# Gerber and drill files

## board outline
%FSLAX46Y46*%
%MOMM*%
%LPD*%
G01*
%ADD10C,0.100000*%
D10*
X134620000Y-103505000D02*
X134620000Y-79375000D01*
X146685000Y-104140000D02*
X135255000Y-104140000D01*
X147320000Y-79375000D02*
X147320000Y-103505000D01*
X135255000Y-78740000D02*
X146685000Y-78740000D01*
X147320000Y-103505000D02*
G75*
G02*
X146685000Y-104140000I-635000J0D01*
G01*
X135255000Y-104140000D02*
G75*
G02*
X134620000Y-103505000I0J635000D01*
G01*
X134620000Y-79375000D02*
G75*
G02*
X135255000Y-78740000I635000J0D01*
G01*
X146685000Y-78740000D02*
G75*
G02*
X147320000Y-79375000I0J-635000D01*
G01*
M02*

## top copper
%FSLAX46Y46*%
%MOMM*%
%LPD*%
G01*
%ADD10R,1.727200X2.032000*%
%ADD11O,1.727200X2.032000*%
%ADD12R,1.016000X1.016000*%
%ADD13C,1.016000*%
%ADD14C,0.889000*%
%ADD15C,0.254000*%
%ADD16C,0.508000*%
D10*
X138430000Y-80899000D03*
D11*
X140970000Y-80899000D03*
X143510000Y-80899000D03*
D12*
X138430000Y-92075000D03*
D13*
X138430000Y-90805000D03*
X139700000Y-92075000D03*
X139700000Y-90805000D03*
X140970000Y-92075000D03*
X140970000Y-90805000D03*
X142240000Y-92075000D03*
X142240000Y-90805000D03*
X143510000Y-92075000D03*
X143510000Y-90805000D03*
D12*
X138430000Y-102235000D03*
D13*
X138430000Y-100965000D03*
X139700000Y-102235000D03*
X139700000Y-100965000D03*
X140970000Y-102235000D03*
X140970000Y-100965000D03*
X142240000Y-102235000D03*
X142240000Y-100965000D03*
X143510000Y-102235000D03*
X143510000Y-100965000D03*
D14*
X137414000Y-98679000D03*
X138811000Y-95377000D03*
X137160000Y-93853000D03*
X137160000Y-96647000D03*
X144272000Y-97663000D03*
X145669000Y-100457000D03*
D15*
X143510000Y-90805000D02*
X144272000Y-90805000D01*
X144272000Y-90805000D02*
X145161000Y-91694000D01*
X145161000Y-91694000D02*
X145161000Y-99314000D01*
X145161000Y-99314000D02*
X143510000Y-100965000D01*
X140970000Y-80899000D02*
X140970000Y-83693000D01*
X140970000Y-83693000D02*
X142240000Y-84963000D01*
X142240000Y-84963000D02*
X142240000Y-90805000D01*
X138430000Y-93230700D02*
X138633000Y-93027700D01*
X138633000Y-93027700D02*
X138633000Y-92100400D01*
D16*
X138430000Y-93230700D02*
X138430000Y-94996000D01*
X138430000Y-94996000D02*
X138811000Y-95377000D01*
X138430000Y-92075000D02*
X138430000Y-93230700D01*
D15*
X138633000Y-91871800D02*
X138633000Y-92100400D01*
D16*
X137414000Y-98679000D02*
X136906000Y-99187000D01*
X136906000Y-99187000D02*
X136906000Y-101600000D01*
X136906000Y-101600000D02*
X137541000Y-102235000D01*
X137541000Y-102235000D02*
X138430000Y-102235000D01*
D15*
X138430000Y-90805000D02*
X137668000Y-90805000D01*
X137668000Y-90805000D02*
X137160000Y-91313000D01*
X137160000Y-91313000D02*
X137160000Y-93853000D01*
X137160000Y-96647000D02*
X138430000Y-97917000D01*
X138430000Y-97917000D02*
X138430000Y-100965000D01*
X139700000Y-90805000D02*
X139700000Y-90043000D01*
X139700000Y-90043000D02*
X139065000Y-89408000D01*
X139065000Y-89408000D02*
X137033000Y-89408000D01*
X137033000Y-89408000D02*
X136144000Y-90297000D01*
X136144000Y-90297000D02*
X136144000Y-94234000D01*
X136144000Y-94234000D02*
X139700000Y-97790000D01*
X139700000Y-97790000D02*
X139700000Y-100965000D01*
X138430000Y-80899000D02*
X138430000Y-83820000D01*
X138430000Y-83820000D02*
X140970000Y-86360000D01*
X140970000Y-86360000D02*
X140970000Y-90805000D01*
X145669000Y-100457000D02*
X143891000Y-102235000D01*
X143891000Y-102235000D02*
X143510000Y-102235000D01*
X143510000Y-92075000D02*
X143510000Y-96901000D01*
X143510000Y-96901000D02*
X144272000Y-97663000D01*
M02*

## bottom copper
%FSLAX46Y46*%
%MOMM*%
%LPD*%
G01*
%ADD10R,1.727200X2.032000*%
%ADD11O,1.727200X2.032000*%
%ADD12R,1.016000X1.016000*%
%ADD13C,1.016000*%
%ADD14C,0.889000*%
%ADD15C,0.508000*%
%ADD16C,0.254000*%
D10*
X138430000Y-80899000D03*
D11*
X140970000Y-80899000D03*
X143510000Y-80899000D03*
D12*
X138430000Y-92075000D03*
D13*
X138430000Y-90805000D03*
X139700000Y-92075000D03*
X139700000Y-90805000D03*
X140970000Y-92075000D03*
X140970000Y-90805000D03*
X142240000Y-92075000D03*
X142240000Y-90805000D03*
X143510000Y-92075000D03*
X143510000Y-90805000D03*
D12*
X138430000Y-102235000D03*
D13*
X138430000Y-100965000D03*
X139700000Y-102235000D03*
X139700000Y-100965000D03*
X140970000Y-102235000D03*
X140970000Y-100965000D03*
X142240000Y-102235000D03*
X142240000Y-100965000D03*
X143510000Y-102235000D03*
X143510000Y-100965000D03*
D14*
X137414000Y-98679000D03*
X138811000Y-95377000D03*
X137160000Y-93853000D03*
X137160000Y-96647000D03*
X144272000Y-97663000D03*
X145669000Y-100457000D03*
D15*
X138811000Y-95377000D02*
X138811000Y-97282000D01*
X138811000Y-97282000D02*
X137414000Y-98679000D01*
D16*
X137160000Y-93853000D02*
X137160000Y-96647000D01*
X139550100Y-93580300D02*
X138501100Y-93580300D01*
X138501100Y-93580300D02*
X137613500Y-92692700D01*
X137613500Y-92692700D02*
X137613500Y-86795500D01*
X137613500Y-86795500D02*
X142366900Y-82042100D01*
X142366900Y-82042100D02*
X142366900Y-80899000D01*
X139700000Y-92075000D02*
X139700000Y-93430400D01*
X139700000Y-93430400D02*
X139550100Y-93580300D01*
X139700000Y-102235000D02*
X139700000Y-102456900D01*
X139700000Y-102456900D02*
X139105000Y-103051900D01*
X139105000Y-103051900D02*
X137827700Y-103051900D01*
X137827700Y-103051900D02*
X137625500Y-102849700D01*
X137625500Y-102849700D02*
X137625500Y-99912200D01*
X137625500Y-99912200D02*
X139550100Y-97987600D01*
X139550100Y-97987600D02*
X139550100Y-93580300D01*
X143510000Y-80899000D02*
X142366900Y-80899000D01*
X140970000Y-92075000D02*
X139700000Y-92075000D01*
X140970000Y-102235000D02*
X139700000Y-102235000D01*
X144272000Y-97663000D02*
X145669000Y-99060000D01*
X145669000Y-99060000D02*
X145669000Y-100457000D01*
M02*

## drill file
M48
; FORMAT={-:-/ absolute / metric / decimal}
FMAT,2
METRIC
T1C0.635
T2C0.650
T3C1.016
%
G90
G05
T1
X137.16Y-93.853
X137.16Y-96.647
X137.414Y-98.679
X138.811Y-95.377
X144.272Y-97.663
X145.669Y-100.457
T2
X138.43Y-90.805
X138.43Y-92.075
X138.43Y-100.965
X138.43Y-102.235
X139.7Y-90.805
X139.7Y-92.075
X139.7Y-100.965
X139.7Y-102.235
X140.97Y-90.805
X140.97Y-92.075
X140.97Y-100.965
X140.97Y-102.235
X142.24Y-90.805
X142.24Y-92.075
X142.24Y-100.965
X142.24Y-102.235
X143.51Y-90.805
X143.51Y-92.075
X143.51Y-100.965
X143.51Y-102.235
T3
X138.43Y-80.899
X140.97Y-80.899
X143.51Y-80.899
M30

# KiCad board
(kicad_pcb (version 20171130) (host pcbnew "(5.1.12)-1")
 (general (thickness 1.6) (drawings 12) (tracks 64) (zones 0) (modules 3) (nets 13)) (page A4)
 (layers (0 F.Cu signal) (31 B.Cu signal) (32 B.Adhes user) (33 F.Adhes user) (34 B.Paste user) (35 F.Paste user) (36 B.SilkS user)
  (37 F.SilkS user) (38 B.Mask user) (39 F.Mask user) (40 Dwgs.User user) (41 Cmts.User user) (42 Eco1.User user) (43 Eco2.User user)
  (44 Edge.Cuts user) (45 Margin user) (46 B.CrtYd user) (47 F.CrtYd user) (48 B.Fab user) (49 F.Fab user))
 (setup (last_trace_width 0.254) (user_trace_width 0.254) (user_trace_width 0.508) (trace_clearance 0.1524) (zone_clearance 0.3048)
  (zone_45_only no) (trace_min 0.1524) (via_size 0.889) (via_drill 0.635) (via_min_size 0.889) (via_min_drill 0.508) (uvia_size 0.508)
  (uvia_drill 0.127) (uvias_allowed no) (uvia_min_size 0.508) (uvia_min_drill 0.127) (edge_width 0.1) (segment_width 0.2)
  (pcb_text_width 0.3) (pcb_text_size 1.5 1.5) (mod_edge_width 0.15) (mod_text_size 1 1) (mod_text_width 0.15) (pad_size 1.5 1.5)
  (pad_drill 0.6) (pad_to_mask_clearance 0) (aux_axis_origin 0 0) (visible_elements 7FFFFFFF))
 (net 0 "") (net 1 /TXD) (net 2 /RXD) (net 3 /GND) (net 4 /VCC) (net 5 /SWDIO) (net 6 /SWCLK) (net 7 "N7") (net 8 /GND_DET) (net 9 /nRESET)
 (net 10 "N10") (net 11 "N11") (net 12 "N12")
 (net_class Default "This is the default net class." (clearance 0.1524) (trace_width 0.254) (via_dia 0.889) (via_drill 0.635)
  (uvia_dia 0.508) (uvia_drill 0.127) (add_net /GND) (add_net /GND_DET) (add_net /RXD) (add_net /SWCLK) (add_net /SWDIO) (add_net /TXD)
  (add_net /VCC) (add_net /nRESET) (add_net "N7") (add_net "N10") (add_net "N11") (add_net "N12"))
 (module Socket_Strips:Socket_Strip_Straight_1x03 (layer F.Cu) (at 140.97 80.899 180)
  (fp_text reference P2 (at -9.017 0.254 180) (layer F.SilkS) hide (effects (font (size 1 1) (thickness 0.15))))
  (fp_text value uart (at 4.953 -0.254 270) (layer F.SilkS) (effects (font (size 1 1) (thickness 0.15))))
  (pad 1 thru_hole rect (at 2.54 0) (size 1.7272 2.032) (drill 1.016) (layers *.Cu *.Mask F.SilkS) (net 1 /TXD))
  (pad 2 thru_hole oval (at 0 0) (size 1.7272 2.032) (drill 1.016) (layers *.Cu *.Mask F.SilkS) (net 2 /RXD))
  (pad 3 thru_hole oval (at -2.54 0) (size 1.7272 2.032) (drill 1.016) (layers *.Cu *.Mask F.SilkS) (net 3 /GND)))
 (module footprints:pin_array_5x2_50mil (layer F.Cu) (at 139.7 91.44)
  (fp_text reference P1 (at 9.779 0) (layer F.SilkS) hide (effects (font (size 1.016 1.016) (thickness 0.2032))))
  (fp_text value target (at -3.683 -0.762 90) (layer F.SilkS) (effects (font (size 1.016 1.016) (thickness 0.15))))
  (pad 1 thru_hole rect (at -1.27 0.635) (size 1.016 1.016) (drill 0.65) (layers *.Cu *.Mask F.SilkS) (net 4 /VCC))
  (pad 2 thru_hole circle (at -1.27 -0.635) (size 1.016 1.016) (drill 0.65) (layers *.Cu *.Mask F.SilkS) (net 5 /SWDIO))
  (pad 3 thru_hole circle (at 0 0.635) (size 1.016 1.016) (drill 0.65) (layers *.Cu *.Mask F.SilkS) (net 3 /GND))
  (pad 4 thru_hole circle (at 0 -0.635) (size 1.016 1.016) (drill 0.65) (layers *.Cu *.Mask F.SilkS) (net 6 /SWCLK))
  (pad 5 thru_hole circle (at 1.27 0.635) (size 1.016 1.016) (drill 0.65) (layers *.Cu *.Mask F.SilkS) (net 3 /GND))
  (pad 6 thru_hole circle (at 1.27 -0.635) (size 1.016 1.016) (drill 0.65) (layers *.Cu *.Mask F.SilkS) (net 1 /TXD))
  (pad 7 thru_hole circle (at 2.54 0.635) (size 1.016 1.016) (drill 0.65) (layers *.Cu *.Mask F.SilkS) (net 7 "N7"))
  (pad 8 thru_hole circle (at 2.54 -0.635) (size 1.016 1.016) (drill 0.65) (layers *.Cu *.Mask F.SilkS) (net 2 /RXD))
  (pad 9 thru_hole circle (at 3.81 0.635) (size 1.016 1.016) (drill 0.65) (layers *.Cu *.Mask F.SilkS) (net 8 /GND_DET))
  (pad 10 thru_hole circle (at 3.81 -0.635) (size 1.016 1.016) (drill 0.65) (layers *.Cu *.Mask F.SilkS) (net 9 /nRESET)))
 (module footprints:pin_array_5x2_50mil (layer F.Cu) (at 139.7 101.6)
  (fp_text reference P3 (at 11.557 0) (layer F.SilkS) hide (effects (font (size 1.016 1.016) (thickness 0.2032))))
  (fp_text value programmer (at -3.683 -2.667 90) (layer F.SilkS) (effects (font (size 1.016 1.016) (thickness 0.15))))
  (pad 1 thru_hole rect (at -1.27 0.635) (size 1.016 1.016) (drill 0.65) (layers *.Cu *.Mask F.SilkS) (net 4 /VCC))
  (pad 2 thru_hole circle (at -1.27 -0.635) (size 1.016 1.016) (drill 0.65) (layers *.Cu *.Mask F.SilkS) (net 5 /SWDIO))
  (pad 3 thru_hole circle (at 0 0.635) (size 1.016 1.016) (drill 0.65) (layers *.Cu *.Mask F.SilkS) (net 3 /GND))
  (pad 4 thru_hole circle (at 0 -0.635) (size 1.016 1.016) (drill 0.65) (layers *.Cu *.Mask F.SilkS) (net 6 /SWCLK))
  (pad 5 thru_hole circle (at 1.27 0.635) (size 1.016 1.016) (drill 0.65) (layers *.Cu *.Mask F.SilkS) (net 3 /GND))
  (pad 6 thru_hole circle (at 1.27 -0.635) (size 1.016 1.016) (drill 0.65) (layers *.Cu *.Mask F.SilkS) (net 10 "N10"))
  (pad 7 thru_hole circle (at 2.54 0.635) (size 1.016 1.016) (drill 0.65) (layers *.Cu *.Mask F.SilkS) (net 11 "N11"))
  (pad 8 thru_hole circle (at 2.54 -0.635) (size 1.016 1.016) (drill 0.65) (layers *.Cu *.Mask F.SilkS) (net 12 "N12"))
  (pad 9 thru_hole circle (at 3.81 0.635) (size 1.016 1.016) (drill 0.65) (layers *.Cu *.Mask F.SilkS) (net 8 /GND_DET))
  (pad 10 thru_hole circle (at 3.81 -0.635) (size 1.016 1.016) (drill 0.65) (layers *.Cu *.Mask F.SilkS) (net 9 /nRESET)))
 (gr_line (start 134.62 103.505) (end 134.62 79.375) (angle 90) (layer Edge.Cuts) (width 0.1))
 (gr_line (start 146.685 104.14) (end 135.255 104.14) (angle 90) (layer Edge.Cuts) (width 0.1))
 (gr_line (start 147.32 79.375) (end 147.32 103.505) (angle 90) (layer Edge.Cuts) (width 0.1))
 (gr_line (start 135.255 78.74) (end 146.685 78.74) (angle 90) (layer Edge.Cuts) (width 0.1))
 (gr_arc (start 146.685 103.505) (end 147.32 103.505) (angle 90) (layer Edge.Cuts) (width 0.1))
 (gr_arc (start 135.255 103.505) (end 135.255 104.14) (angle 90) (layer Edge.Cuts) (width 0.1))
 (gr_arc (start 135.255 79.375) (end 134.62 79.375) (angle 90) (layer Edge.Cuts) (width 0.1))
 (gr_arc (start 146.685 79.375) (end 146.685 78.74) (angle 90) (layer Edge.Cuts) (width 0.1))
 (segment (start 143.51 90.805) (end 144.272 90.805) (width 0.254) (layer F.Cu) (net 9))
 (segment (start 144.272 90.805) (end 145.161 91.694) (width 0.254) (layer F.Cu) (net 9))
 (segment (start 145.161 91.694) (end 145.161 99.314) (width 0.254) (layer F.Cu) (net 9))
 (segment (start 145.161 99.314) (end 143.51 100.965) (width 0.254) (layer F.Cu) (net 9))
 (segment (start 140.97 80.899) (end 140.97 83.693) (width 0.254) (layer F.Cu) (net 2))
 (segment (start 140.97 83.693) (end 142.24 84.963) (width 0.254) (layer F.Cu) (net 2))
 (segment (start 142.24 84.963) (end 142.24 90.805) (width 0.254) (layer F.Cu) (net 2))
 (segment (start 138.43 93.2307) (end 138.633 93.0277) (width 0.254) (layer F.Cu) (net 4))
 (segment (start 138.633 93.0277) (end 138.633 92.1004) (width 0.254) (layer F.Cu) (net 4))
 (segment (start 138.43 93.2307) (end 138.43 94.996) (width 0.508) (layer F.Cu) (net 4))
 (segment (start 138.43 94.996) (end 138.811 95.377) (width 0.508) (layer F.Cu) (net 4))
 (segment (start 138.43 92.075) (end 138.43 93.2307) (width 0.508) (layer F.Cu) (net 4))
 (segment (start 138.633 91.8718) (end 138.633 92.1004) (width 0.254) (layer F.Cu) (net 4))
 (segment (start 137.414 98.679) (end 136.906 99.187) (width 0.508) (layer F.Cu) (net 4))
 (segment (start 136.906 99.187) (end 136.906 101.6) (width 0.508) (layer F.Cu) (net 4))
 (segment (start 136.906 101.6) (end 137.541 102.235) (width 0.508) (layer F.Cu) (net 4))
 (segment (start 137.541 102.235) (end 138.43 102.235) (width 0.508) (layer F.Cu) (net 4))
 (segment (start 138.811 95.377) (end 138.811 97.282) (width 0.508) (layer B.Cu) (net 4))
 (segment (start 138.811 97.282) (end 137.414 98.679) (width 0.508) (layer B.Cu) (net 4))
 (via (at 137.414 98.679) (size 0.889) (layers F.Cu B.Cu) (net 4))
 (via (at 138.811 95.377) (size 0.889) (layers F.Cu B.Cu) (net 4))
 (segment (start 138.43 90.805) (end 137.668 90.805) (width 0.254) (layer F.Cu) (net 5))
 (segment (start 137.668 90.805) (end 137.16 91.313) (width 0.254) (layer F.Cu) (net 5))
 (segment (start 137.16 91.313) (end 137.16 93.853) (width 0.254) (layer F.Cu) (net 5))
 (segment (start 137.16 93.853) (end 137.16 96.647) (width 0.254) (layer B.Cu) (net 5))
 (segment (start 137.16 96.647) (end 138.43 97.917) (width 0.254) (layer F.Cu) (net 5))
 (segment (start 138.43 97.917) (end 138.43 100.965) (width 0.254) (layer F.Cu) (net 5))
 (via (at 137.16 93.853) (size 0.889) (layers F.Cu B.Cu) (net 5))
 (via (at 137.16 96.647) (size 0.889) (layers F.Cu B.Cu) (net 5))
 (segment (start 139.5501 93.5803) (end 138.5011 93.5803) (width 0.254) (layer B.Cu) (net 3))
 (segment (start 138.5011 93.5803) (end 137.6135 92.6927) (width 0.254) (layer B.Cu) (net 3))
 (segment (start 137.6135 92.6927) (end 137.6135 86.7955) (width 0.254) (layer B.Cu) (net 3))
 (segment (start 137.6135 86.7955) (end 142.3669 82.0421) (width 0.254) (layer B.Cu) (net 3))
 (segment (start 142.3669 82.0421) (end 142.3669 80.899) (width 0.254) (layer B.Cu) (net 3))
 (segment (start 139.7 92.075) (end 139.7 93.4304) (width 0.254) (layer B.Cu) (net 3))
 (segment (start 139.7 93.4304) (end 139.5501 93.5803) (width 0.254) (layer B.Cu) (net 3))
 (segment (start 139.7 102.235) (end 139.7 102.4569) (width 0.254) (layer B.Cu) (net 3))
 (segment (start 139.7 102.4569) (end 139.105 103.0519) (width 0.254) (layer B.Cu) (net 3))
 (segment (start 139.105 103.0519) (end 137.8277 103.0519) (width 0.254) (layer B.Cu) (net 3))
 (segment (start 137.8277 103.0519) (end 137.6255 102.8497) (width 0.254) (layer B.Cu) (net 3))
 (segment (start 137.6255 102.8497) (end 137.6255 99.9122) (width 0.254) (layer B.Cu) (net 3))
 (segment (start 137.6255 99.9122) (end 139.5501 97.9876) (width 0.254) (layer B.Cu) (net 3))
 (segment (start 139.5501 97.9876) (end 139.5501 93.5803) (width 0.254) (layer B.Cu) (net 3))
 (segment (start 143.51 80.899) (end 142.3669 80.899) (width 0.254) (layer B.Cu) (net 3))
 (segment (start 140.97 92.075) (end 139.7 92.075) (width 0.254) (layer B.Cu) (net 3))
 (segment (start 140.97 102.235) (end 139.7 102.235) (width 0.254) (layer B.Cu) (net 3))
 (segment (start 139.7 90.805) (end 139.7 90.043) (width 0.254) (layer F.Cu) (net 6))
 (segment (start 139.7 90.043) (end 139.065 89.408) (width 0.254) (layer F.Cu) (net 6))
 (segment (start 139.065 89.408) (end 137.033 89.408) (width 0.254) (layer F.Cu) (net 6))
 (segment (start 137.033 89.408) (end 136.144 90.297) (width 0.254) (layer F.Cu) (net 6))
 (segment (start 136.144 90.297) (end 136.144 94.234) (width 0.254) (layer F.Cu) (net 6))
 (segment (start 136.144 94.234) (end 139.7 97.79) (width 0.254) (layer F.Cu) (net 6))
 (segment (start 139.7 97.79) (end 139.7 100.965) (width 0.254) (layer F.Cu) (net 6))
 (segment (start 138.43 80.899) (end 138.43 83.82) (width 0.254) (layer F.Cu) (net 1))
 (segment (start 138.43 83.82) (end 140.97 86.36) (width 0.254) (layer F.Cu) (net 1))
 (segment (start 140.97 86.36) (end 140.97 90.805) (width 0.254) (layer F.Cu) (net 1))
 (segment (start 145.669 100.457) (end 143.891 102.235) (width 0.254) (layer F.Cu) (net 8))
 (segment (start 143.891 102.235) (end 143.51 102.235) (width 0.254) (layer F.Cu) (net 8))
 (segment (start 143.51 92.075) (end 143.51 96.901) (width 0.254) (layer F.Cu) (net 8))
 (segment (start 143.51 96.901) (end 144.272 97.663) (width 0.254) (layer F.Cu) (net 8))
 (segment (start 144.272 97.663) (end 145.669 99.06) (width 0.254) (layer B.Cu) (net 8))
 (segment (start 145.669 99.06) (end 145.669 100.457) (width 0.254) (layer B.Cu) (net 8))
 (via (at 144.272 97.663) (size 0.889) (layers F.Cu B.Cu) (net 8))
 (via (at 145.669 100.457) (size 0.889) (layers F.Cu B.Cu) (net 8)))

